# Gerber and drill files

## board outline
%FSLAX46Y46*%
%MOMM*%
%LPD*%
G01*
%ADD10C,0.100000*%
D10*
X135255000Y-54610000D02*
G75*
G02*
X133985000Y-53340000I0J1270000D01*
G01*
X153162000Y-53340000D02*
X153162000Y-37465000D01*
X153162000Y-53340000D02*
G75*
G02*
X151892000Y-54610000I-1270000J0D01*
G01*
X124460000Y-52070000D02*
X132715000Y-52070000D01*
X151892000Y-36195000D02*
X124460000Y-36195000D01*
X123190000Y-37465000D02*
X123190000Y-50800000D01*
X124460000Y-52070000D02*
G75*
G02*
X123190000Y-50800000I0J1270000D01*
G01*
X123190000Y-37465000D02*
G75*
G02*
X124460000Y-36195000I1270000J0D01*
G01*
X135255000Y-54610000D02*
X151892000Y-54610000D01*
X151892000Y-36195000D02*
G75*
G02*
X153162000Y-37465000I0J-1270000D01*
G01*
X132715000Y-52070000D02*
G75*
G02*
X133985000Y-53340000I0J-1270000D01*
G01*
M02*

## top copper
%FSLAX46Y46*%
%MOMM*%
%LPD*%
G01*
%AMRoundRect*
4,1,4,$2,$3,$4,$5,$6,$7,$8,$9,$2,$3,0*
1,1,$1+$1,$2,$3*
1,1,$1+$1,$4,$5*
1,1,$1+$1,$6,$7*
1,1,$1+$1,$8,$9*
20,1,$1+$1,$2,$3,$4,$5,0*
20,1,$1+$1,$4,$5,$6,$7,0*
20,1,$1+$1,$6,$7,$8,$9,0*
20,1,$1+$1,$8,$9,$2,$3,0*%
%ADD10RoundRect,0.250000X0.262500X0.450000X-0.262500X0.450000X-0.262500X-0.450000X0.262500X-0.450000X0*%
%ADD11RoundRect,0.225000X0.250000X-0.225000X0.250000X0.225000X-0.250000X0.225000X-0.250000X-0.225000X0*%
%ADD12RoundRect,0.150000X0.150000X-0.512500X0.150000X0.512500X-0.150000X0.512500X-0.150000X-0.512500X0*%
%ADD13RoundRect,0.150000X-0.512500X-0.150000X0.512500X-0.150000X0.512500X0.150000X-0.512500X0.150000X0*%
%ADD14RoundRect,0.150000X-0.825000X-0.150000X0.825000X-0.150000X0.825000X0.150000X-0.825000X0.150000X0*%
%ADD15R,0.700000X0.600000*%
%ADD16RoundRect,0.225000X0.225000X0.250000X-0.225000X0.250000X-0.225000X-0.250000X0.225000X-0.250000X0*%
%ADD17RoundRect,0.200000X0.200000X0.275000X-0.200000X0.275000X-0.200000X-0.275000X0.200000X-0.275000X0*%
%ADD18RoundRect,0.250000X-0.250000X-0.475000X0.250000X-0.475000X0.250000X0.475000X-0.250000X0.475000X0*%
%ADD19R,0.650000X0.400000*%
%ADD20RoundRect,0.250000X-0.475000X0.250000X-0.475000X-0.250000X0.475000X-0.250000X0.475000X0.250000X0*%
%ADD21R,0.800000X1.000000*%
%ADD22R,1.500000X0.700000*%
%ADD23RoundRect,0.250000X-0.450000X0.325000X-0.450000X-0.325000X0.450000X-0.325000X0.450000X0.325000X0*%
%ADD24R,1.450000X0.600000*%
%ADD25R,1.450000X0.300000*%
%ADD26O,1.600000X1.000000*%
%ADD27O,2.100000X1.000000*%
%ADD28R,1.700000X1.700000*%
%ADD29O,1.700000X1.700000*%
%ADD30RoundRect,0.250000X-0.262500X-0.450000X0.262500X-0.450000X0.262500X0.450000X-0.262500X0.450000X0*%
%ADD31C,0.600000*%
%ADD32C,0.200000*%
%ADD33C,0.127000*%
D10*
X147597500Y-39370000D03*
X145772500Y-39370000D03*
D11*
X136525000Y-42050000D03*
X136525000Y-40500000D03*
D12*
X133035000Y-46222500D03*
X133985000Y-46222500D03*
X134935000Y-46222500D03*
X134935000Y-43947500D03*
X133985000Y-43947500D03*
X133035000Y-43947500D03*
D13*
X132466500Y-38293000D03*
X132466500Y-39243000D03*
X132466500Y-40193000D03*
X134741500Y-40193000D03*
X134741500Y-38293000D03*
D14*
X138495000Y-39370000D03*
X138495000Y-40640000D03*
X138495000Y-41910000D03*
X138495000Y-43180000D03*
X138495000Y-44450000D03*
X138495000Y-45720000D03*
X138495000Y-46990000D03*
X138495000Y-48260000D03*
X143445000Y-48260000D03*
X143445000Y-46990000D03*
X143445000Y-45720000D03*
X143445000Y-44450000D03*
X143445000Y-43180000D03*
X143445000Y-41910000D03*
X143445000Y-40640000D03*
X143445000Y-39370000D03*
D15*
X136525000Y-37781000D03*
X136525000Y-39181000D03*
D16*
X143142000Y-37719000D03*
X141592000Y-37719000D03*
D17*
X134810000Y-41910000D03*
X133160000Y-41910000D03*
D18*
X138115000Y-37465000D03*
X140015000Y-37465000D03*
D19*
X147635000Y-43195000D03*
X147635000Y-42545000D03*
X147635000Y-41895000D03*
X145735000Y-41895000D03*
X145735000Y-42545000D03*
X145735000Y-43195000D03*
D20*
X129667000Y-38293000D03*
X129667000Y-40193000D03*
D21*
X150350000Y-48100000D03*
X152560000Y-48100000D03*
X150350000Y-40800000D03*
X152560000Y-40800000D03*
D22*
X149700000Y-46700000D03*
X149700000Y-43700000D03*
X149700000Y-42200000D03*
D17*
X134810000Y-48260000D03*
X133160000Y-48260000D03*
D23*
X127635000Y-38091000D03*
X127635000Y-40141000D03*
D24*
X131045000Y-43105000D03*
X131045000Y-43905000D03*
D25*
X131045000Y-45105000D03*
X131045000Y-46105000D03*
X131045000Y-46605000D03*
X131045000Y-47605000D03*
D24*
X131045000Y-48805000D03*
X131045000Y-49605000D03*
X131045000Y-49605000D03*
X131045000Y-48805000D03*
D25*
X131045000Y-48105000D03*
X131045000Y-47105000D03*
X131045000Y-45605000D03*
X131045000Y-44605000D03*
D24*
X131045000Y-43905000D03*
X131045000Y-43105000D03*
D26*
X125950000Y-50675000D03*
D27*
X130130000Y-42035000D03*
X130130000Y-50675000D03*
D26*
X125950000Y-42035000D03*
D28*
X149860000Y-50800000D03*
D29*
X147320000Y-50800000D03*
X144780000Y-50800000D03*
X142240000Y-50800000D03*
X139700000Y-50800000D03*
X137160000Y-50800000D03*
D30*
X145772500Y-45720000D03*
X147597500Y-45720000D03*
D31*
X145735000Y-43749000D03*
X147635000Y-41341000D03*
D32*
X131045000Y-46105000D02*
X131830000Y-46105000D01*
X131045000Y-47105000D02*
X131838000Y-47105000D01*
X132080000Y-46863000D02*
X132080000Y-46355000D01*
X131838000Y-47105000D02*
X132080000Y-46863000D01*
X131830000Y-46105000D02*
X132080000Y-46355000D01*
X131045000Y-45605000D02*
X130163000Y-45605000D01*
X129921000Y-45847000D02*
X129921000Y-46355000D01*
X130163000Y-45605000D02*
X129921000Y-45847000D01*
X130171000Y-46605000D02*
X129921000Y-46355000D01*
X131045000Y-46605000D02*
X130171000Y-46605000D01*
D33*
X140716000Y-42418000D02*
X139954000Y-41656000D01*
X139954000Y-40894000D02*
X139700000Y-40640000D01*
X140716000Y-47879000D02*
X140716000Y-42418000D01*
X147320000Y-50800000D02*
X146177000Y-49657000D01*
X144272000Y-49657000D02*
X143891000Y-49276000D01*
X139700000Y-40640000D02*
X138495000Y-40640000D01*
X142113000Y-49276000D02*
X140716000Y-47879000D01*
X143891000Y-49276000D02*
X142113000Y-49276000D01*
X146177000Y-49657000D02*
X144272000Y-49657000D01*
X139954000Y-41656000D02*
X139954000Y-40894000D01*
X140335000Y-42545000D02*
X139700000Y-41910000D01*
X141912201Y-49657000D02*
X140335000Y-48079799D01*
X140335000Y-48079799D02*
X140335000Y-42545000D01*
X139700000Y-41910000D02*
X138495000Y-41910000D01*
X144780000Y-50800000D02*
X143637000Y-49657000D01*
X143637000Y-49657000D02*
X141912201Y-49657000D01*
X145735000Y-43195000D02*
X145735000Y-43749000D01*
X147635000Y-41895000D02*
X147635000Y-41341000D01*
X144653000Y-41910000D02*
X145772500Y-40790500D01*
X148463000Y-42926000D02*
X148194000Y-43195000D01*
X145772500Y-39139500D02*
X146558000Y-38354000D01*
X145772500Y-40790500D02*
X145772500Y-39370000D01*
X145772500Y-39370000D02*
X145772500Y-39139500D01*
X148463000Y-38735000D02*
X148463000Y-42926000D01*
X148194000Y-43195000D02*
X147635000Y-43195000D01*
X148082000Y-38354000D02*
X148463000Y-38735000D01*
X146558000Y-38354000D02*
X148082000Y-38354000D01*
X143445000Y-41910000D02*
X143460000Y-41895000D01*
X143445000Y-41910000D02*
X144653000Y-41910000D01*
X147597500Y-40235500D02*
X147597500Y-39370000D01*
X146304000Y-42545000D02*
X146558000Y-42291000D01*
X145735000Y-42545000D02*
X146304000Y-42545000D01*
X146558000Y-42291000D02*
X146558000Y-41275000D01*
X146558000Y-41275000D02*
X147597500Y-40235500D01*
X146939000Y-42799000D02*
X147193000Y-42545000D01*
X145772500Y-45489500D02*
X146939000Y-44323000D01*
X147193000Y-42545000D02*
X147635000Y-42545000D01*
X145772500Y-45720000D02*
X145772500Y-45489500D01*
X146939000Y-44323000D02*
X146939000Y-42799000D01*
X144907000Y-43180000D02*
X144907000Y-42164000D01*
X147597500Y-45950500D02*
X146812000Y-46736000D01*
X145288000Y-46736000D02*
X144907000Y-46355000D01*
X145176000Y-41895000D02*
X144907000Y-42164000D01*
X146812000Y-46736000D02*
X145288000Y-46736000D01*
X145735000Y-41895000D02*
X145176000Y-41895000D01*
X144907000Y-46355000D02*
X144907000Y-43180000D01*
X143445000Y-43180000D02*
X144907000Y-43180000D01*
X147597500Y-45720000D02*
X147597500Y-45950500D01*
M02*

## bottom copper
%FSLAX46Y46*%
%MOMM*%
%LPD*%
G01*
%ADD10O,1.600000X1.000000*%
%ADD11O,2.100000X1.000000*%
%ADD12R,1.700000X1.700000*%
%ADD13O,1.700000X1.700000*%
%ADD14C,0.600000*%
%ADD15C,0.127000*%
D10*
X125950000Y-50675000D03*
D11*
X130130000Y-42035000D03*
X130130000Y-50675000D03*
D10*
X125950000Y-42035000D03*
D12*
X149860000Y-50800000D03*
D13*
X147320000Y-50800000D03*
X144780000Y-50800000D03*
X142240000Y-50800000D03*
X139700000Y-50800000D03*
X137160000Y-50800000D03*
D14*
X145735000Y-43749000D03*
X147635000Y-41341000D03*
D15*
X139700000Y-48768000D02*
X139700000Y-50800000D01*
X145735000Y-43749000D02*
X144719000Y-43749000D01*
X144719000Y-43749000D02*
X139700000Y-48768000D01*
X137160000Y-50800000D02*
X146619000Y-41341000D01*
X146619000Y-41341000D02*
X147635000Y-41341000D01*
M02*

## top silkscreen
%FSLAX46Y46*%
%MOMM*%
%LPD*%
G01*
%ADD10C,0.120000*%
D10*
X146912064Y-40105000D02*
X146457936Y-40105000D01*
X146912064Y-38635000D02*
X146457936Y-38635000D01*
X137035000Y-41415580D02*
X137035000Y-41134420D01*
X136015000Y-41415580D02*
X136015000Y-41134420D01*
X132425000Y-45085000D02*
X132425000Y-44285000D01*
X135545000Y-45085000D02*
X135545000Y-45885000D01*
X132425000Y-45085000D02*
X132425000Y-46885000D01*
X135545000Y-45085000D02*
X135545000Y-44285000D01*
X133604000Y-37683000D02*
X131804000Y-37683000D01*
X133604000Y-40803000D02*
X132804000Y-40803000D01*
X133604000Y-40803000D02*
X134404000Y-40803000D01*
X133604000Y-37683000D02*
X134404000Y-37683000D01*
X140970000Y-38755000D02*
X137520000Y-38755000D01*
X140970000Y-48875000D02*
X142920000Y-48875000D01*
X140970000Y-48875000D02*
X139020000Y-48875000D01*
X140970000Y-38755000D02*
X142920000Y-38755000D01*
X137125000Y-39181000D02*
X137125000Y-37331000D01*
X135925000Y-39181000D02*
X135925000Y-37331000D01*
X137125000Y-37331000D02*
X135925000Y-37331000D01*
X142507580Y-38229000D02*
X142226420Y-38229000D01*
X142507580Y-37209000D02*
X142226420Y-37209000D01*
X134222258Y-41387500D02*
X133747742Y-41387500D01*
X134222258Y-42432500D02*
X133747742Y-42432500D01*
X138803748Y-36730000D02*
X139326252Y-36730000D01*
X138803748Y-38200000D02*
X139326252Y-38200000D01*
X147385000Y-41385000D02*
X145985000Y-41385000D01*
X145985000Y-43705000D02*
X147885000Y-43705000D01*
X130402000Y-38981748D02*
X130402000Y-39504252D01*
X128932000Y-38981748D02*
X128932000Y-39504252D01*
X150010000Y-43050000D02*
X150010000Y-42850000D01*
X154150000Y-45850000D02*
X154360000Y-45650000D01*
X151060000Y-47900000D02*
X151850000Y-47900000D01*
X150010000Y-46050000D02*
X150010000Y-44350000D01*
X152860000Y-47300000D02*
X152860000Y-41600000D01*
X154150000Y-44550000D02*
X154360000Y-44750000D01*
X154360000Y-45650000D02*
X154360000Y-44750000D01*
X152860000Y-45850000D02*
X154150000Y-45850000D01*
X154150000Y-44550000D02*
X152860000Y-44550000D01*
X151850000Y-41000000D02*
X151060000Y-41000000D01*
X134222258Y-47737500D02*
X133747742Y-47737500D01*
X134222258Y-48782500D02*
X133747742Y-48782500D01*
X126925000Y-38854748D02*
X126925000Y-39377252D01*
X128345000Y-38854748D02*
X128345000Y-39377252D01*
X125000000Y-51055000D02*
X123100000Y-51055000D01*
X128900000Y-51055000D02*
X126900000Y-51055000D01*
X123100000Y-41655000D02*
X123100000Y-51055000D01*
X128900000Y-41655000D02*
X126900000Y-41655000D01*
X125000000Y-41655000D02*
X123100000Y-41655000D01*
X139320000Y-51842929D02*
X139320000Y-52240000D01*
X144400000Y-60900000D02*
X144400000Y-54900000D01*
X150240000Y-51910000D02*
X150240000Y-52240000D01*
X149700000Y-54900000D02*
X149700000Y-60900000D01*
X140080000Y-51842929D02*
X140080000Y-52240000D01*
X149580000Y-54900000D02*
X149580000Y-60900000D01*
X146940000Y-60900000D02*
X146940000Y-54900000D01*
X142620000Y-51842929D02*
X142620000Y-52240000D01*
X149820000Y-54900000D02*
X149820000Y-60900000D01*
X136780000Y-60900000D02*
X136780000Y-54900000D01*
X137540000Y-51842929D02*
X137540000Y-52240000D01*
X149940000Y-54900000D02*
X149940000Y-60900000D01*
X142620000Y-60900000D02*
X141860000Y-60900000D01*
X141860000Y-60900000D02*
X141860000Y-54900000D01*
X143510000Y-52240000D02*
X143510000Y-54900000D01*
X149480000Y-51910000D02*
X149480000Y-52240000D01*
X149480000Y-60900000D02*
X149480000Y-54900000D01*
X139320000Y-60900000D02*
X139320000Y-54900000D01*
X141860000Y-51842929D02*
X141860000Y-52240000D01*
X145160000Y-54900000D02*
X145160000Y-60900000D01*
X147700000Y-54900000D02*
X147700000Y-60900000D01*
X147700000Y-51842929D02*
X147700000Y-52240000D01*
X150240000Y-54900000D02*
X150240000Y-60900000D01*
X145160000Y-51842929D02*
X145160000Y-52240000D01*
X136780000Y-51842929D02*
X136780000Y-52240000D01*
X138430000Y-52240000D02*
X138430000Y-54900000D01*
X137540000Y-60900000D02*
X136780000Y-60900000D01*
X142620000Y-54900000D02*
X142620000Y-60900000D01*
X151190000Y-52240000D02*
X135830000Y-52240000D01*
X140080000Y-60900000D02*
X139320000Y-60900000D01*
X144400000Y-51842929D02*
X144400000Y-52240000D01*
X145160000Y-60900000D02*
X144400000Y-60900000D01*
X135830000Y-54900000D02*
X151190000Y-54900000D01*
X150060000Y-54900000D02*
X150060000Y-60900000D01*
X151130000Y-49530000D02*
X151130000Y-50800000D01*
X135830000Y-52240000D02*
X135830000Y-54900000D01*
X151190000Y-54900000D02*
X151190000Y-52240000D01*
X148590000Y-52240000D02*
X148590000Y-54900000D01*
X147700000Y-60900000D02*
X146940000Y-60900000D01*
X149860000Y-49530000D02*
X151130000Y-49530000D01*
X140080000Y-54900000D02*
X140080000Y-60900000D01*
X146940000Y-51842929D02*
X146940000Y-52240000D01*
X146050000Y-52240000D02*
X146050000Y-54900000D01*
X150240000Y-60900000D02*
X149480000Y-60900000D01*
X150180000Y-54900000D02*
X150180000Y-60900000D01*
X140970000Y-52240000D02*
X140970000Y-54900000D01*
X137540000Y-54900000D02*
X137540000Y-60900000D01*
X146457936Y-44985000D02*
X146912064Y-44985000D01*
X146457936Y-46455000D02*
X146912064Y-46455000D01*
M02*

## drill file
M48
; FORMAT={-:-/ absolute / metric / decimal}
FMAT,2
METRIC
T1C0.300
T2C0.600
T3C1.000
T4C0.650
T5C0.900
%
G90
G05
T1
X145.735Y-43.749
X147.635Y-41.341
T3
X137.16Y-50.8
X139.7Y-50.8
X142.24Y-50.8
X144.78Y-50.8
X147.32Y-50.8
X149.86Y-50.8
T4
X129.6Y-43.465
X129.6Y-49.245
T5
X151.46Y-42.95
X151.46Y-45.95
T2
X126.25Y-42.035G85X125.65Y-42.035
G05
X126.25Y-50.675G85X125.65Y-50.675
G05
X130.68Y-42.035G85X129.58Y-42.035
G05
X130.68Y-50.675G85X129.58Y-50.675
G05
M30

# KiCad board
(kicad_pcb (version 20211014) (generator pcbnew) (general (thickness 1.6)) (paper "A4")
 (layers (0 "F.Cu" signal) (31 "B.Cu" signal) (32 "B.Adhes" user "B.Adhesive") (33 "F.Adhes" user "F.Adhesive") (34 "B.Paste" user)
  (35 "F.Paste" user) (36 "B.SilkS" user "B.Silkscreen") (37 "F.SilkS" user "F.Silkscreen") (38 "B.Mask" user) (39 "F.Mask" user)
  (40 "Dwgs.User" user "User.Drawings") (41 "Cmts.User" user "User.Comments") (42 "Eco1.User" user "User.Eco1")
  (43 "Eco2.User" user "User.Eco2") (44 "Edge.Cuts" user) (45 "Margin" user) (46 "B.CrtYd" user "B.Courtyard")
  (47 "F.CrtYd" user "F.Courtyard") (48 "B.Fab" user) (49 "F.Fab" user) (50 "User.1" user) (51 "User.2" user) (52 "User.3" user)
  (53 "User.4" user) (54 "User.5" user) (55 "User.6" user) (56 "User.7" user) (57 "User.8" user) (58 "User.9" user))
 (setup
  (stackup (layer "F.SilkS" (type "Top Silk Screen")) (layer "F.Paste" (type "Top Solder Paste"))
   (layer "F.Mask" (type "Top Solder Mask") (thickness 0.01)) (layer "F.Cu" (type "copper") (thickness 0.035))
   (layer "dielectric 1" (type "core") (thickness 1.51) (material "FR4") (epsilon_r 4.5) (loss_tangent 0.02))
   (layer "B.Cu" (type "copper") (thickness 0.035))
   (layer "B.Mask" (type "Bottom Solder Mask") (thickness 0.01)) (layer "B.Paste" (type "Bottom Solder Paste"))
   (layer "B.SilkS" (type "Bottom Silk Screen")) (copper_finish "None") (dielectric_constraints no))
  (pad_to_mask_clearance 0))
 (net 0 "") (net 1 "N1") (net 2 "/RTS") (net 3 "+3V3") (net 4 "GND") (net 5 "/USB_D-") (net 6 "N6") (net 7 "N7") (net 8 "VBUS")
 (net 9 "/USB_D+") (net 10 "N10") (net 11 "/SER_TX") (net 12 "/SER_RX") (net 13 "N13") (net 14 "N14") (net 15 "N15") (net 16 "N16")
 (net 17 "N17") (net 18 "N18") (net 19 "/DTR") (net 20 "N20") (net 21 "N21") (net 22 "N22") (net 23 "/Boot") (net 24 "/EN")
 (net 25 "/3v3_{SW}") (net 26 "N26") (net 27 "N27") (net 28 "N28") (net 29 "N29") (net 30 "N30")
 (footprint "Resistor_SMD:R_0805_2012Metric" (layer "F.Cu") (at 146.685 39.37 180)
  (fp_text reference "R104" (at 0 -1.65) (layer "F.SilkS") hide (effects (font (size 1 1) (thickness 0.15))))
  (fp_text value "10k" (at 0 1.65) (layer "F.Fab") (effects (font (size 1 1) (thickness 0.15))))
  (fp_line (start -0.227064 -0.735) (end 0.227064 -0.735) (layer "F.SilkS") (width 0.12))
  (fp_line (start -0.227064 0.735) (end 0.227064 0.735) (layer "F.SilkS") (width 0.12))
  (pad "1" smd roundrect locked (at -0.9125 0 180) (size 1.025 1.4) (layers "F.Cu" "F.Paste" "F.Mask") (roundrect_rratio 0.243902)
   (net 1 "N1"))
  (pad "2" smd roundrect locked (at 0.9125 0 180) (size 1.025 1.4) (layers "F.Cu" "F.Paste" "F.Mask") (roundrect_rratio 0.243902)
   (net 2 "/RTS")))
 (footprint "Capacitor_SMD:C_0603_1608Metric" (layer "F.Cu") (at 136.525 41.275 90) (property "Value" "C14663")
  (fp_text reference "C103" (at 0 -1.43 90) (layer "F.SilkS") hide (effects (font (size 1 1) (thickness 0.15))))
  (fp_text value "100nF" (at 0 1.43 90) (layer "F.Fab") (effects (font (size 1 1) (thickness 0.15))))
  (fp_line (start -0.14058 0.51) (end 0.14058 0.51) (layer "F.SilkS") (width 0.12))
  (fp_line (start -0.14058 -0.51) (end 0.14058 -0.51) (layer "F.SilkS") (width 0.12))
  (pad "1" smd roundrect locked (at -0.775 0 90) (size 0.9 0.95) (layers "F.Cu" "F.Paste" "F.Mask") (roundrect_rratio 0.25) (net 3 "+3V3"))
  (pad "2" smd roundrect locked (at 0.775 0 90) (size 0.9 0.95) (layers "F.Cu" "F.Paste" "F.Mask") (roundrect_rratio 0.25) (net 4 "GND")))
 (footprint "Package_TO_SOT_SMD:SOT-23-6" (layer "F.Cu") (at 133.985 45.085 90)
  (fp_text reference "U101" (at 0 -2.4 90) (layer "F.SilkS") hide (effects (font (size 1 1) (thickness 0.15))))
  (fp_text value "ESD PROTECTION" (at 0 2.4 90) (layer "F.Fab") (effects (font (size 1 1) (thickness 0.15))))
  (fp_line (start 0 -1.56) (end 0.8 -1.56) (layer "F.SilkS") (width 0.12))
  (fp_line (start 0 1.56) (end -0.8 1.56) (layer "F.SilkS") (width 0.12))
  (fp_line (start 0 -1.56) (end -1.8 -1.56) (layer "F.SilkS") (width 0.12))
  (fp_line (start 0 1.56) (end 0.8 1.56) (layer "F.SilkS") (width 0.12))
  (pad "1" smd roundrect locked (at -1.1375 -0.95 90) (size 1.325 0.6) (layers "F.Cu" "F.Paste" "F.Mask") (roundrect_rratio 0.25)
   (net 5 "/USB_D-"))
  (pad "2" smd roundrect locked (at -1.1375 0 90) (size 1.325 0.6) (layers "F.Cu" "F.Paste" "F.Mask") (roundrect_rratio 0.25) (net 4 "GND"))
  (pad "3" smd roundrect locked (at -1.1375 0.95 90) (size 1.325 0.6) (layers "F.Cu" "F.Paste" "F.Mask") (roundrect_rratio 0.25)
   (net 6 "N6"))
  (pad "4" smd roundrect locked (at 1.1375 0.95 90) (size 1.325 0.6) (layers "F.Cu" "F.Paste" "F.Mask") (roundrect_rratio 0.25) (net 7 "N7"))
  (pad "5" smd roundrect locked (at 1.1375 0 90) (size 1.325 0.6) (layers "F.Cu" "F.Paste" "F.Mask") (roundrect_rratio 0.25) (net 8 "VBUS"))
  (pad "6" smd roundrect locked (at 1.1375 -0.95 90) (size 1.325 0.6) (layers "F.Cu" "F.Paste" "F.Mask") (roundrect_rratio 0.25)
   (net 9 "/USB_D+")))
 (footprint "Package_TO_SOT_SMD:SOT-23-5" (layer "F.Cu") (at 133.604 39.243)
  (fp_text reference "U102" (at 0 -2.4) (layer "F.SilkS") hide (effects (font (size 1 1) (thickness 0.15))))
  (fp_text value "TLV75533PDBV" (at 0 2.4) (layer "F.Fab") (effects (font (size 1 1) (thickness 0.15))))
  (fp_line (start 0 -1.56) (end -1.8 -1.56) (layer "F.SilkS") (width 0.12))
  (fp_line (start 0 1.56) (end -0.8 1.56) (layer "F.SilkS") (width 0.12))
  (fp_line (start 0 1.56) (end 0.8 1.56) (layer "F.SilkS") (width 0.12))
  (fp_line (start 0 -1.56) (end 0.8 -1.56) (layer "F.SilkS") (width 0.12))
  (pad "1" smd roundrect locked (at -1.1375 -0.95) (size 1.325 0.6) (layers "F.Cu" "F.Paste" "F.Mask") (roundrect_rratio 0.25)
   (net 8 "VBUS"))
  (pad "2" smd roundrect locked (at -1.1375 0) (size 1.325 0.6) (layers "F.Cu" "F.Paste" "F.Mask") (roundrect_rratio 0.25) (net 4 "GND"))
  (pad "3" smd roundrect locked (at -1.1375 0.95) (size 1.325 0.6) (layers "F.Cu" "F.Paste" "F.Mask") (roundrect_rratio 0.25) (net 8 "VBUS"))
  (pad "4" smd roundrect locked (at 1.1375 0.95) (size 1.325 0.6) (layers "F.Cu" "F.Paste" "F.Mask") (roundrect_rratio 0.25) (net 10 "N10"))
  (pad "5" smd roundrect locked (at 1.1375 -0.95) (size 1.325 0.6) (layers "F.Cu" "F.Paste" "F.Mask") (roundrect_rratio 0.25) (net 3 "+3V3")))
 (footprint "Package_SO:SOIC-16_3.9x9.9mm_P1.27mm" (layer "F.Cu") (at 140.97 43.815)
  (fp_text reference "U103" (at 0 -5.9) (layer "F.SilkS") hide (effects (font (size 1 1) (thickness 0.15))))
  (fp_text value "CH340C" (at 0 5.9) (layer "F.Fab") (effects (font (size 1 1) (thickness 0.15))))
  (fp_line (start 0 -5.06) (end -3.45 -5.06) (layer "F.SilkS") (width 0.12))
  (fp_line (start 0 5.06) (end 1.95 5.06) (layer "F.SilkS") (width 0.12))
  (fp_line (start 0 5.06) (end -1.95 5.06) (layer "F.SilkS") (width 0.12))
  (fp_line (start 0 -5.06) (end 1.95 -5.06) (layer "F.SilkS") (width 0.12))
  (pad "1" smd roundrect locked (at -2.475 -4.445) (size 1.95 0.6) (layers "F.Cu" "F.Paste" "F.Mask") (roundrect_rratio 0.25) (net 4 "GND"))
  (pad "2" smd roundrect locked (at -2.475 -3.175) (size 1.95 0.6) (layers "F.Cu" "F.Paste" "F.Mask") (roundrect_rratio 0.25)
   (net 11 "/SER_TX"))
  (pad "3" smd roundrect locked (at -2.475 -1.905) (size 1.95 0.6) (layers "F.Cu" "F.Paste" "F.Mask") (roundrect_rratio 0.25)
   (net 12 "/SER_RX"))
  (pad "4" smd roundrect locked (at -2.475 -0.635) (size 1.95 0.6) (layers "F.Cu" "F.Paste" "F.Mask") (roundrect_rratio 0.25) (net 3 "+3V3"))
  (pad "5" smd roundrect locked (at -2.475 0.635) (size 1.95 0.6) (layers "F.Cu" "F.Paste" "F.Mask") (roundrect_rratio 0.25)
   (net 9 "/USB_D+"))
  (pad "6" smd roundrect locked (at -2.475 1.905) (size 1.95 0.6) (layers "F.Cu" "F.Paste" "F.Mask") (roundrect_rratio 0.25)
   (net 5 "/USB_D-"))
  (pad "7" smd roundrect locked (at -2.475 3.175) (size 1.95 0.6) (layers "F.Cu" "F.Paste" "F.Mask") (roundrect_rratio 0.25) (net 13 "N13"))
  (pad "8" smd roundrect locked (at -2.475 4.445) (size 1.95 0.6) (layers "F.Cu" "F.Paste" "F.Mask") (roundrect_rratio 0.25) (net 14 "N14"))
  (pad "9" smd roundrect locked (at 2.475 4.445) (size 1.95 0.6) (layers "F.Cu" "F.Paste" "F.Mask") (roundrect_rratio 0.25) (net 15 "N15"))
  (pad "10" smd roundrect locked (at 2.475 3.175) (size 1.95 0.6) (layers "F.Cu" "F.Paste" "F.Mask") (roundrect_rratio 0.25) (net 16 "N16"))
  (pad "11" smd roundrect locked (at 2.475 1.905) (size 1.95 0.6) (layers "F.Cu" "F.Paste" "F.Mask") (roundrect_rratio 0.25) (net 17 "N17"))
  (pad "12" smd roundrect locked (at 2.475 0.635) (size 1.95 0.6) (layers "F.Cu" "F.Paste" "F.Mask") (roundrect_rratio 0.25) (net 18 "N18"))
  (pad "13" smd roundrect locked (at 2.475 -0.635) (size 1.95 0.6) (layers "F.Cu" "F.Paste" "F.Mask") (roundrect_rratio 0.25)
   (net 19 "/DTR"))
  (pad "14" smd roundrect locked (at 2.475 -1.905) (size 1.95 0.6) (layers "F.Cu" "F.Paste" "F.Mask") (roundrect_rratio 0.25) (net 2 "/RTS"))
  (pad "15" smd roundrect locked (at 2.475 -3.175) (size 1.95 0.6) (layers "F.Cu" "F.Paste" "F.Mask") (roundrect_rratio 0.25) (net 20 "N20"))
  (pad "16" smd roundrect locked (at 2.475 -4.445) (size 1.95 0.6) (layers "F.Cu" "F.Paste" "F.Mask") (roundrect_rratio 0.25) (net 3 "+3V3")))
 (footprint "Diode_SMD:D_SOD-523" (layer "F.Cu") (at 136.525 38.481 -90)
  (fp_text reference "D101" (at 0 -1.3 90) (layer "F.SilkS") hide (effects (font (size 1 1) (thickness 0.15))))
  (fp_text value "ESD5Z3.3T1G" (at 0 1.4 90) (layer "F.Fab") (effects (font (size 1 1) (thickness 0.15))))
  (fp_line (start 0.7 -0.6) (end -1.15 -0.6) (layer "F.SilkS") (width 0.12))
  (fp_line (start 0.7 0.6) (end -1.15 0.6) (layer "F.SilkS") (width 0.12))
  (fp_line (start -1.15 -0.6) (end -1.15 0.6) (layer "F.SilkS") (width 0.12))
  (pad "1" smd rect locked (at -0.7 0 90) (size 0.6 0.7) (layers "F.Cu" "F.Paste" "F.Mask") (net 3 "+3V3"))
  (pad "2" smd rect locked (at 0.7 0 90) (size 0.6 0.7) (layers "F.Cu" "F.Paste" "F.Mask") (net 4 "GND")))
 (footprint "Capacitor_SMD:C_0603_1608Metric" (layer "F.Cu") (at 142.367 37.719 180) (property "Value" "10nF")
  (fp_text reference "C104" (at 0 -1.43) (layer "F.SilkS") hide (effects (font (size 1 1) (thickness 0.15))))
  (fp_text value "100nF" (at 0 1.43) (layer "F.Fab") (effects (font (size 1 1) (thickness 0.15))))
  (fp_line (start -0.14058 -0.51) (end 0.14058 -0.51) (layer "F.SilkS") (width 0.12))
  (fp_line (start -0.14058 0.51) (end 0.14058 0.51) (layer "F.SilkS") (width 0.12))
  (pad "1" smd roundrect locked (at -0.775 0 180) (size 0.9 0.95) (layers "F.Cu" "F.Paste" "F.Mask") (roundrect_rratio 0.25) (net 3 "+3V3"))
  (pad "2" smd roundrect locked (at 0.775 0 180) (size 0.9 0.95) (layers "F.Cu" "F.Paste" "F.Mask") (roundrect_rratio 0.25) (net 4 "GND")))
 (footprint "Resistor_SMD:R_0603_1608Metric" (layer "F.Cu") (at 133.985 41.91 180)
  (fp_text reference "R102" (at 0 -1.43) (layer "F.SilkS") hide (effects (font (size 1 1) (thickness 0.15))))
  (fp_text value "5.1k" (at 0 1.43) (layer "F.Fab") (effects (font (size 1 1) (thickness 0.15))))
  (fp_line (start -0.237258 0.5225) (end 0.237258 0.5225) (layer "F.SilkS") (width 0.12))
  (fp_line (start -0.237258 -0.5225) (end 0.237258 -0.5225) (layer "F.SilkS") (width 0.12))
  (pad "1" smd roundrect locked (at -0.825 0 180) (size 0.8 0.95) (layers "F.Cu" "F.Paste" "F.Mask") (roundrect_rratio 0.25) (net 4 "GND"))
  (pad "2" smd roundrect locked (at 0.825 0 180) (size 0.8 0.95) (layers "F.Cu" "F.Paste" "F.Mask") (roundrect_rratio 0.25) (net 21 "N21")))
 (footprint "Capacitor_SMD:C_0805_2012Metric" (layer "F.Cu") (at 139.065 37.465)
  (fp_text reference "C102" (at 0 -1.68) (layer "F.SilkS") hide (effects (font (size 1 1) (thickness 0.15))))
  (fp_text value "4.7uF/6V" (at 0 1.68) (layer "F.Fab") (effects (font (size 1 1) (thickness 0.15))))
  (fp_line (start -0.261252 -0.735) (end 0.261252 -0.735) (layer "F.SilkS") (width 0.12))
  (fp_line (start -0.261252 0.735) (end 0.261252 0.735) (layer "F.SilkS") (width 0.12))
  (pad "1" smd roundrect locked (at -0.95 0) (size 1 1.45) (layers "F.Cu" "F.Paste" "F.Mask") (roundrect_rratio 0.25) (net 3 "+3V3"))
  (pad "2" smd roundrect locked (at 0.95 0) (size 1 1.45) (layers "F.Cu" "F.Paste" "F.Mask") (roundrect_rratio 0.25) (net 4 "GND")))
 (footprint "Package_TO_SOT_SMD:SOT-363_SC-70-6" (layer "F.Cu") (at 146.685 42.545 180)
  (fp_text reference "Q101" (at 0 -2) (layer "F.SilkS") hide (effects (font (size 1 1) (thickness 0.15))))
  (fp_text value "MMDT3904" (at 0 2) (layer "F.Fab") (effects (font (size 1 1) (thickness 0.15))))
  (fp_line (start -0.7 1.16) (end 0.7 1.16) (layer "F.SilkS") (width 0.12))
  (fp_line (start 0.7 -1.16) (end -1.2 -1.16) (layer "F.SilkS") (width 0.12))
  (pad "1" smd rect locked (at -0.95 -0.65 180) (size 0.65 0.4) (layers "F.Cu" "F.Paste" "F.Mask") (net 2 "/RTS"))
  (pad "2" smd rect locked (at -0.95 0 180) (size 0.65 0.4) (layers "F.Cu" "F.Paste" "F.Mask") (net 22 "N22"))
  (pad "3" smd rect locked (at -0.95 0.65 180) (size 0.65 0.4) (layers "F.Cu" "F.Paste" "F.Mask") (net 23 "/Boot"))
  (pad "4" smd rect locked (at 0.95 0.65 180) (size 0.65 0.4) (layers "F.Cu" "F.Paste" "F.Mask") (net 19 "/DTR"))
  (pad "5" smd rect locked (at 0.95 0 180) (size 0.65 0.4) (layers "F.Cu" "F.Paste" "F.Mask") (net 1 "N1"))
  (pad "6" smd rect locked (at 0.95 -0.65 180) (size 0.65 0.4) (layers "F.Cu" "F.Paste" "F.Mask") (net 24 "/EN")))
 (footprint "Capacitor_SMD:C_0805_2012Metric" (layer "F.Cu") (at 129.667 39.243 -90)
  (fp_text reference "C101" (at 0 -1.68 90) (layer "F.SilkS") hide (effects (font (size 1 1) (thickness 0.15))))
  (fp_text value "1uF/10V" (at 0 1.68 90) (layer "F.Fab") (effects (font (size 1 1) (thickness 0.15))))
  (fp_line (start -0.261252 -0.735) (end 0.261252 -0.735) (layer "F.SilkS") (width 0.12))
  (fp_line (start -0.261252 0.735) (end 0.261252 0.735) (layer "F.SilkS") (width 0.12))
  (pad "1" smd roundrect locked (at -0.95 0 270) (size 1 1.45) (layers "F.Cu" "F.Paste" "F.Mask") (roundrect_rratio 0.25) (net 8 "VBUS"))
  (pad "2" smd roundrect locked (at 0.95 0 270) (size 1 1.45) (layers "F.Cu" "F.Paste" "F.Mask") (roundrect_rratio 0.25) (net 4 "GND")))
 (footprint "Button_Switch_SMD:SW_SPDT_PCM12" (layer "F.Cu") (at 151.13 44.45 90)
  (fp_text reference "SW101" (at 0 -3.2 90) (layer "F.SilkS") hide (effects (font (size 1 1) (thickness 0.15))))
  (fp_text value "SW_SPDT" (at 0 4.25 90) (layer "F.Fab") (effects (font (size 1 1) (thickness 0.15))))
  (fp_line (start 1.4 -1.12) (end 1.6 -1.12) (layer "F.SilkS") (width 0.12))
  (fp_line (start -1.4 3.02) (end -1.2 3.23) (layer "F.SilkS") (width 0.12))
  (fp_line (start -3.45 -0.07) (end -3.45 0.72) (layer "F.SilkS") (width 0.12))
  (fp_line (start -1.6 -1.12) (end 0.1 -1.12) (layer "F.SilkS") (width 0.12))
  (fp_line (start -2.85 1.73) (end 2.85 1.73) (layer "F.SilkS") (width 0.12))
  (fp_line (start -0.1 3.02) (end -0.3 3.23) (layer "F.SilkS") (width 0.12))
  (fp_line (start -1.2 3.23) (end -0.3 3.23) (layer "F.SilkS") (width 0.12))
  (fp_line (start -1.4 1.73) (end -1.4 3.02) (layer "F.SilkS") (width 0.12))
  (fp_line (start -0.1 3.02) (end -0.1 1.73) (layer "F.SilkS") (width 0.12))
  (fp_line (start 3.45 0.72) (end 3.45 -0.07) (layer "F.SilkS") (width 0.12))
  (pad "" smd rect locked (at -3.65 -0.78 90) (size 1 0.8) (layers "F.Cu" "F.Paste" "F.Mask"))
  (pad "" np_thru_hole circle locked (at -1.5 0.33 90) (size 0.9 0.9) (drill 0.9) (layers *.Cu *.Mask))
  (pad "" smd rect locked (at -3.65 1.43 90) (size 1 0.8) (layers "F.Cu" "F.Paste" "F.Mask"))
  (pad "" smd rect locked (at 3.65 -0.78 90) (size 1 0.8) (layers "F.Cu" "F.Paste" "F.Mask"))
  (pad "" smd rect locked (at 3.65 1.43 90) (size 1 0.8) (layers "F.Cu" "F.Paste" "F.Mask"))
  (pad "" np_thru_hole circle locked (at 1.5 0.33 90) (size 0.9 0.9) (drill 0.9) (layers *.Cu *.Mask))
  (pad "1" smd rect locked (at -2.25 -1.43 90) (size 0.7 1.5) (layers "F.Cu" "F.Paste" "F.Mask") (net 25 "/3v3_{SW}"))
  (pad "2" smd rect locked (at 0.75 -1.43 90) (size 0.7 1.5) (layers "F.Cu" "F.Paste" "F.Mask") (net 3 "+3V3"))
  (pad "3" smd rect locked (at 2.25 -1.43 90) (size 0.7 1.5) (layers "F.Cu" "F.Paste" "F.Mask") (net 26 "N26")))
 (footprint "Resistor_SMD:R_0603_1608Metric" (layer "F.Cu") (at 133.985 48.26 180)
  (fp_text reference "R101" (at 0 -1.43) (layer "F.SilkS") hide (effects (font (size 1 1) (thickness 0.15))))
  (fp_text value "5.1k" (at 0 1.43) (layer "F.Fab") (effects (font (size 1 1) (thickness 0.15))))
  (fp_line (start -0.237258 0.5225) (end 0.237258 0.5225) (layer "F.SilkS") (width 0.12))
  (fp_line (start -0.237258 -0.5225) (end 0.237258 -0.5225) (layer "F.SilkS") (width 0.12))
  (pad "1" smd roundrect locked (at -0.825 0 180) (size 0.8 0.95) (layers "F.Cu" "F.Paste" "F.Mask") (roundrect_rratio 0.25) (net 4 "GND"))
  (pad "2" smd roundrect locked (at 0.825 0 180) (size 0.8 0.95) (layers "F.Cu" "F.Paste" "F.Mask") (roundrect_rratio 0.25) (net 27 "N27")))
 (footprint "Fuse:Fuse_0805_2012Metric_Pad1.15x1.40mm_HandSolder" (layer "F.Cu") (at 127.635 39.116 -90)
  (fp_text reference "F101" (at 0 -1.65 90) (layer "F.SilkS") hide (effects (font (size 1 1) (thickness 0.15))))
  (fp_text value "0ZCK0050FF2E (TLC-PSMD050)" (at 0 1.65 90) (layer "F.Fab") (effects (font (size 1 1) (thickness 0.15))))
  (fp_line (start -0.261252 0.71) (end 0.261252 0.71) (layer "F.SilkS") (width 0.12))
  (fp_line (start -0.261252 -0.71) (end 0.261252 -0.71) (layer "F.SilkS") (width 0.12))
  (pad "1" smd roundrect locked (at -1.025 0 270) (size 1.15 1.4) (layers "F.Cu" "F.Paste" "F.Mask") (roundrect_rratio 0.217391)
   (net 8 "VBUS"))
  (pad "2" smd roundrect locked (at 1.025 0 270) (size 1.15 1.4) (layers "F.Cu" "F.Paste" "F.Mask") (roundrect_rratio 0.217391)
   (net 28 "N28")))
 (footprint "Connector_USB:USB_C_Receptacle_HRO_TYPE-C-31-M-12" (layer "F.Cu") (at 127 46.355 -90)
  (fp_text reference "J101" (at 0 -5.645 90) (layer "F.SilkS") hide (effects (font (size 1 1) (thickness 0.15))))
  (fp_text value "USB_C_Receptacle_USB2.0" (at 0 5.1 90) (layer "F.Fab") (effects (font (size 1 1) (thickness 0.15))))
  (fp_line (start 4.7 2) (end 4.7 3.9) (layer "F.SilkS") (width 0.12))
  (fp_line (start 4.7 -1.9) (end 4.7 0.1) (layer "F.SilkS") (width 0.12))
  (fp_line (start -4.7 3.9) (end 4.7 3.9) (layer "F.SilkS") (width 0.12))
  (fp_line (start -4.7 -1.9) (end -4.7 0.1) (layer "F.SilkS") (width 0.12))
  (fp_line (start -4.7 2) (end -4.7 3.9) (layer "F.SilkS") (width 0.12))
  (pad "" np_thru_hole circle locked (at 2.89 -2.6 270) (size 0.65 0.65) (drill 0.65) (layers *.Cu *.Mask))
  (pad "" np_thru_hole circle locked (at -2.89 -2.6 270) (size 0.65 0.65) (drill 0.65) (layers *.Cu *.Mask))
  (pad "A1" smd rect locked (at -3.25 -4.045 270) (size 0.6 1.45) (layers "F.Cu" "F.Paste" "F.Mask") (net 4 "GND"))
  (pad "A4" smd rect locked (at -2.45 -4.045 270) (size 0.6 1.45) (layers "F.Cu" "F.Paste" "F.Mask") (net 28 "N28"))
  (pad "A5" smd rect locked (at -1.25 -4.045 270) (size 0.3 1.45) (layers "F.Cu" "F.Paste" "F.Mask") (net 21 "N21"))
  (pad "A6" smd rect locked (at -0.25 -4.045 270) (size 0.3 1.45) (layers "F.Cu" "F.Paste" "F.Mask") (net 9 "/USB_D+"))
  (pad "A7" smd rect locked (at 0.25 -4.045 270) (size 0.3 1.45) (layers "F.Cu" "F.Paste" "F.Mask") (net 5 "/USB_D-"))
  (pad "A8" smd rect locked (at 1.25 -4.045 270) (size 0.3 1.45) (layers "F.Cu" "F.Paste" "F.Mask") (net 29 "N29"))
  (pad "A9" smd rect locked (at 2.45 -4.045 270) (size 0.6 1.45) (layers "F.Cu" "F.Paste" "F.Mask") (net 28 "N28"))
  (pad "A12" smd rect locked (at 3.25 -4.045 270) (size 0.6 1.45) (layers "F.Cu" "F.Paste" "F.Mask") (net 4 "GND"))
  (pad "B1" smd rect locked (at 3.25 -4.045 270) (size 0.6 1.45) (layers "F.Cu" "F.Paste" "F.Mask") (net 4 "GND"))
  (pad "B4" smd rect locked (at 2.45 -4.045 270) (size 0.6 1.45) (layers "F.Cu" "F.Paste" "F.Mask") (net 28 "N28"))
  (pad "B5" smd rect locked (at 1.75 -4.045 270) (size 0.3 1.45) (layers "F.Cu" "F.Paste" "F.Mask") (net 27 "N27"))
  (pad "B6" smd rect locked (at 0.75 -4.045 270) (size 0.3 1.45) (layers "F.Cu" "F.Paste" "F.Mask") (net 9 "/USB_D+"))
  (pad "B7" smd rect locked (at -0.75 -4.045 270) (size 0.3 1.45) (layers "F.Cu" "F.Paste" "F.Mask") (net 5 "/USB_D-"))
  (pad "B8" smd rect locked (at -1.75 -4.045 270) (size 0.3 1.45) (layers "F.Cu" "F.Paste" "F.Mask") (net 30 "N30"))
  (pad "B9" smd rect locked (at -2.45 -4.045 270) (size 0.6 1.45) (layers "F.Cu" "F.Paste" "F.Mask") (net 28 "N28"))
  (pad "B12" smd rect locked (at -3.25 -4.045 270) (size 0.6 1.45) (layers "F.Cu" "F.Paste" "F.Mask") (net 4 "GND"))
  (pad "S1" thru_hole oval locked (at 4.32 1.05 270) (size 1 1.6) (drill oval 0.6 1.2) (layers *.Cu *.Mask) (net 4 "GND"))
  (pad "S1" thru_hole oval locked (at -4.32 -3.13 270) (size 1 2.1) (drill oval 0.6 1.7) (layers *.Cu *.Mask) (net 4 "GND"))
  (pad "S1" thru_hole oval locked (at 4.32 -3.13 270) (size 1 2.1) (drill oval 0.6 1.7) (layers *.Cu *.Mask) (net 4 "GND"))
  (pad "S1" thru_hole oval locked (at -4.32 1.05 270) (size 1 1.6) (drill oval 0.6 1.2) (layers *.Cu *.Mask) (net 4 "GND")))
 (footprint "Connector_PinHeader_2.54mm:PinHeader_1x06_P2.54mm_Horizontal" (layer "F.Cu") (at 149.86 50.8 -90)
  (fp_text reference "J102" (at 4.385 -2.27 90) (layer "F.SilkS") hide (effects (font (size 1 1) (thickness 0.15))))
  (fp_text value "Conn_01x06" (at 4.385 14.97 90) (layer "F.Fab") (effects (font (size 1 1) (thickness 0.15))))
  (fp_line (start 1.042929 10.54) (end 1.44 10.54) (layer "F.SilkS") (width 0.12))
  (fp_line (start 10.1 5.46) (end 4.1 5.46) (layer "F.SilkS") (width 0.12))
  (fp_line (start 1.11 -0.38) (end 1.44 -0.38) (layer "F.SilkS") (width 0.12))
  (fp_line (start 4.1 0.16) (end 10.1 0.16) (layer "F.SilkS") (width 0.12))
  (fp_line (start 1.042929 9.78) (end 1.44 9.78) (layer "F.SilkS") (width 0.12))
  (fp_line (start 4.1 0.28) (end 10.1 0.28) (layer "F.SilkS") (width 0.12))
  (fp_line (start 10.1 2.92) (end 4.1 2.92) (layer "F.SilkS") (width 0.12))
  (fp_line (start 1.042929 7.24) (end 1.44 7.24) (layer "F.SilkS") (width 0.12))
  (fp_line (start 4.1 0.04) (end 10.1 0.04) (layer "F.SilkS") (width 0.12))
  (fp_line (start 10.1 13.08) (end 4.1 13.08) (layer "F.SilkS") (width 0.12))
  (fp_line (start 1.042929 12.32) (end 1.44 12.32) (layer "F.SilkS") (width 0.12))
  (fp_line (start 4.1 -0.08) (end 10.1 -0.08) (layer "F.SilkS") (width 0.12))
  (fp_line (start 10.1 7.24) (end 10.1 8) (layer "F.SilkS") (width 0.12))
  (fp_line (start 10.1 8) (end 4.1 8) (layer "F.SilkS") (width 0.12))
  (fp_line (start 1.44 6.35) (end 4.1 6.35) (layer "F.SilkS") (width 0.12))
  (fp_line (start 1.11 0.38) (end 1.44 0.38) (layer "F.SilkS") (width 0.12))
  (fp_line (start 10.1 0.38) (end 4.1 0.38) (layer "F.SilkS") (width 0.12))
  (fp_line (start 10.1 10.54) (end 4.1 10.54) (layer "F.SilkS") (width 0.12))
  (fp_line (start 1.042929 8) (end 1.44 8) (layer "F.SilkS") (width 0.12))
  (fp_line (start 4.1 4.7) (end 10.1 4.7) (layer "F.SilkS") (width 0.12))
  (fp_line (start 4.1 2.16) (end 10.1 2.16) (layer "F.SilkS") (width 0.12))
  (fp_line (start 1.042929 2.16) (end 1.44 2.16) (layer "F.SilkS") (width 0.12))
  (fp_line (start 4.1 -0.38) (end 10.1 -0.38) (layer "F.SilkS") (width 0.12))
  (fp_line (start 1.042929 4.7) (end 1.44 4.7) (layer "F.SilkS") (width 0.12))
  (fp_line (start 1.042929 13.08) (end 1.44 13.08) (layer "F.SilkS") (width 0.12))
  (fp_line (start 1.44 11.43) (end 4.1 11.43) (layer "F.SilkS") (width 0.12))
  (fp_line (start 10.1 12.32) (end 10.1 13.08) (layer "F.SilkS") (width 0.12))
  (fp_line (start 4.1 7.24) (end 10.1 7.24) (layer "F.SilkS") (width 0.12))
  (fp_line (start 1.44 -1.33) (end 1.44 14.03) (layer "F.SilkS") (width 0.12))
  (fp_line (start 10.1 9.78) (end 10.1 10.54) (layer "F.SilkS") (width 0.12))
  (fp_line (start 1.042929 5.46) (end 1.44 5.46) (layer "F.SilkS") (width 0.12))
  (fp_line (start 10.1 4.7) (end 10.1 5.46) (layer "F.SilkS") (width 0.12))
  (fp_line (start 4.1 14.03) (end 4.1 -1.33) (layer "F.SilkS") (width 0.12))
  (fp_line (start 4.1 -0.2) (end 10.1 -0.2) (layer "F.SilkS") (width 0.12))
  (fp_line (start -1.27 -1.27) (end 0 -1.27) (layer "F.SilkS") (width 0.12))
  (fp_line (start 1.44 14.03) (end 4.1 14.03) (layer "F.SilkS") (width 0.12))
  (fp_line (start 4.1 -1.33) (end 1.44 -1.33) (layer "F.SilkS") (width 0.12))
  (fp_line (start 1.44 1.27) (end 4.1 1.27) (layer "F.SilkS") (width 0.12))
  (fp_line (start 10.1 2.16) (end 10.1 2.92) (layer "F.SilkS") (width 0.12))
  (fp_line (start -1.27 0) (end -1.27 -1.27) (layer "F.SilkS") (width 0.12))
  (fp_line (start 4.1 9.78) (end 10.1 9.78) (layer "F.SilkS") (width 0.12))
  (fp_line (start 1.042929 2.92) (end 1.44 2.92) (layer "F.SilkS") (width 0.12))
  (fp_line (start 1.44 3.81) (end 4.1 3.81) (layer "F.SilkS") (width 0.12))
  (fp_line (start 10.1 -0.38) (end 10.1 0.38) (layer "F.SilkS") (width 0.12))
  (fp_line (start 4.1 -0.32) (end 10.1 -0.32) (layer "F.SilkS") (width 0.12))
  (fp_line (start 1.44 8.89) (end 4.1 8.89) (layer "F.SilkS") (width 0.12))
  (fp_line (start 4.1 12.32) (end 10.1 12.32) (layer "F.SilkS") (width 0.12))
  (pad "1" thru_hole rect locked (at 0 0 270) (size 1.7 1.7) (drill 1) (layers *.Cu *.Mask) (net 4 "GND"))
  (pad "2" thru_hole oval locked (at 0 2.54 270) (size 1.7 1.7) (drill 1) (layers *.Cu *.Mask) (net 11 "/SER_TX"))
  (pad "3" thru_hole oval locked (at 0 5.08 270) (size 1.7 1.7) (drill 1) (layers *.Cu *.Mask) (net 12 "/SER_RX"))
  (pad "4" thru_hole oval locked (at 0 7.62 270) (size 1.7 1.7) (drill 1) (layers *.Cu *.Mask) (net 25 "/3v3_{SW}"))
  (pad "5" thru_hole oval locked (at 0 10.16 270) (size 1.7 1.7) (drill 1) (layers *.Cu *.Mask) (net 24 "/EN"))
  (pad "6" thru_hole oval locked (at 0 12.7 270) (size 1.7 1.7) (drill 1) (layers *.Cu *.Mask) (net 23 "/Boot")))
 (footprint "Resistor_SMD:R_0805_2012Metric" (layer "F.Cu") (at 146.685 45.72)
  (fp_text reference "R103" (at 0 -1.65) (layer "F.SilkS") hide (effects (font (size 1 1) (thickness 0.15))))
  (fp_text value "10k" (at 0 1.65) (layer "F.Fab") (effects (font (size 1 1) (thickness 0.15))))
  (fp_line (start -0.227064 -0.735) (end 0.227064 -0.735) (layer "F.SilkS") (width 0.12))
  (fp_line (start -0.227064 0.735) (end 0.227064 0.735) (layer "F.SilkS") (width 0.12))
  (pad "1" smd roundrect locked (at -0.9125 0) (size 1.025 1.4) (layers "F.Cu" "F.Paste" "F.Mask") (roundrect_rratio 0.243902)
   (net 22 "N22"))
  (pad "2" smd roundrect locked (at 0.9125 0) (size 1.025 1.4) (layers "F.Cu" "F.Paste" "F.Mask") (roundrect_rratio 0.243902)
   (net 19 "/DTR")))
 (gr_arc (start 135.255 54.61) (mid 134.356974 54.238026) (end 133.985 53.34) (layer "Edge.Cuts") (width 0.1))
 (gr_line (start 153.162 53.34) (end 153.162 37.465) (layer "Edge.Cuts") (width 0.1))
 (gr_arc (start 153.162 53.34) (mid 152.790026 54.238026) (end 151.892 54.61) (layer "Edge.Cuts") (width 0.1))
 (gr_line (start 124.46 52.07) (end 132.715 52.07) (layer "Edge.Cuts") (width 0.1))
 (gr_line (start 151.892 36.195) (end 124.46 36.195) (layer "Edge.Cuts") (width 0.1))
 (gr_line (start 123.19 37.465) (end 123.19 50.8) (layer "Edge.Cuts") (width 0.1))
 (gr_arc (start 124.46 52.07) (mid 123.561974 51.698026) (end 123.19 50.8) (layer "Edge.Cuts") (width 0.1))
 (gr_arc (start 123.19 37.465) (mid 123.561974 36.566974) (end 124.46 36.195) (layer "Edge.Cuts") (width 0.1))
 (gr_line (start 135.255 54.61) (end 151.892 54.61) (layer "Edge.Cuts") (width 0.1))
 (gr_arc (start 151.892 36.195) (mid 152.790026 36.566974) (end 153.162 37.465) (layer "Edge.Cuts") (width 0.1))
 (gr_arc (start 132.715 52.07) (mid 133.613026 52.441974) (end 133.985 53.34) (layer "Edge.Cuts") (width 0.1))
 (segment (start 131.045 46.105) (end 131.83 46.105) (width 0.2) (layer "F.Cu") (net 9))
 (segment (start 131.045 47.105) (end 131.838 47.105) (width 0.2) (layer "F.Cu") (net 9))
 (segment (start 132.08 46.863) (end 132.08 46.355) (width 0.2) (layer "F.Cu") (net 9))
 (segment (start 131.838 47.105) (end 132.08 46.863) (width 0.2) (layer "F.Cu") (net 9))
 (segment (start 131.83 46.105) (end 132.08 46.355) (width 0.2) (layer "F.Cu") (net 9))
 (segment (start 131.045 45.605) (end 130.163 45.605) (width 0.2) (layer "F.Cu") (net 5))
 (segment (start 129.921 45.847) (end 129.921 46.355) (width 0.2) (layer "F.Cu") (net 5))
 (segment (start 130.163 45.605) (end 129.921 45.847) (width 0.2) (layer "F.Cu") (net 5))
 (segment (start 130.171 46.605) (end 129.921 46.355) (width 0.2) (layer "F.Cu") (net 5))
 (segment (start 131.045 46.605) (end 130.171 46.605) (width 0.2) (layer "F.Cu") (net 5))
 (segment (start 140.716 42.418) (end 139.954 41.656) (width 0.127) (layer "F.Cu") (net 11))
 (segment (start 139.954 40.894) (end 139.7 40.64) (width 0.127) (layer "F.Cu") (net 11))
 (segment (start 140.716 47.879) (end 140.716 42.418) (width 0.127) (layer "F.Cu") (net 11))
 (segment (start 147.32 50.8) (end 146.177 49.657) (width 0.127) (layer "F.Cu") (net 11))
 (segment (start 144.272 49.657) (end 143.891 49.276) (width 0.127) (layer "F.Cu") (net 11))
 (segment (start 139.7 40.64) (end 138.495 40.64) (width 0.127) (layer "F.Cu") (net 11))
 (segment (start 142.113 49.276) (end 140.716 47.879) (width 0.127) (layer "F.Cu") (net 11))
 (segment (start 143.891 49.276) (end 142.113 49.276) (width 0.127) (layer "F.Cu") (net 11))
 (segment (start 146.177 49.657) (end 144.272 49.657) (width 0.127) (layer "F.Cu") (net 11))
 (segment (start 139.954 41.656) (end 139.954 40.894) (width 0.127) (layer "F.Cu") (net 11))
 (segment (start 140.335 42.545) (end 139.7 41.91) (width 0.127) (layer "F.Cu") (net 12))
 (segment (start 141.912201 49.657) (end 140.335 48.079799) (width 0.127) (layer "F.Cu") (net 12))
 (segment (start 140.335 48.079799) (end 140.335 42.545) (width 0.127) (layer "F.Cu") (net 12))
 (segment (start 139.7 41.91) (end 138.495 41.91) (width 0.127) (layer "F.Cu") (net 12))
 (segment (start 144.78 50.8) (end 143.637 49.657) (width 0.127) (layer "F.Cu") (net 12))
 (segment (start 143.637 49.657) (end 141.912201 49.657) (width 0.127) (layer "F.Cu") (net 12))
 (segment (start 145.735 43.195) (end 145.735 43.749) (width 0.127) (layer "F.Cu") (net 24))
 (via (at 145.735 43.749) (size 0.6) (drill 0.3) (layers "F.Cu" "B.Cu") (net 24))
 (segment (start 139.7 48.768) (end 139.7 50.8) (width 0.127) (layer "B.Cu") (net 24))
 (segment (start 145.735 43.749) (end 144.719 43.749) (width 0.127) (layer "B.Cu") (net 24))
 (segment (start 144.719 43.749) (end 139.7 48.768) (width 0.127) (layer "B.Cu") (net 24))
 (segment (start 147.635 41.895) (end 147.635 41.341) (width 0.127) (layer "F.Cu") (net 23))
 (via (at 147.635 41.341) (size 0.6) (drill 0.3) (layers "F.Cu" "B.Cu") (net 23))
 (segment (start 137.16 50.8) (end 146.619 41.341) (width 0.127) (layer "B.Cu") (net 23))
 (segment (start 146.619 41.341) (end 147.635 41.341) (width 0.127) (layer "B.Cu") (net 23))
 (segment (start 144.653 41.91) (end 145.7725 40.7905) (width 0.127) (layer "F.Cu") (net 2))
 (segment (start 148.463 42.926) (end 148.194 43.195) (width 0.127) (layer "F.Cu") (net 2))
 (segment (start 145.7725 39.1395) (end 146.558 38.354) (width 0.127) (layer "F.Cu") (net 2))
 (segment (start 145.7725 40.7905) (end 145.7725 39.37) (width 0.127) (layer "F.Cu") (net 2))
 (segment (start 145.7725 39.37) (end 145.7725 39.1395) (width 0.127) (layer "F.Cu") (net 2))
 (segment (start 148.463 38.735) (end 148.463 42.926) (width 0.127) (layer "F.Cu") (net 2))
 (segment (start 148.194 43.195) (end 147.635 43.195) (width 0.127) (layer "F.Cu") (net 2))
 (segment (start 148.082 38.354) (end 148.463 38.735) (width 0.127) (layer "F.Cu") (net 2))
 (segment (start 146.558 38.354) (end 148.082 38.354) (width 0.127) (layer "F.Cu") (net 2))
 (segment (start 143.445 41.91) (end 143.46 41.895) (width 0.127) (layer "F.Cu") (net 2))
 (segment (start 143.445 41.91) (end 144.653 41.91) (width 0.127) (layer "F.Cu") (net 2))
 (segment (start 147.5975 40.2355) (end 147.5975 39.37) (width 0.127) (layer "F.Cu") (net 1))
 (segment (start 146.304 42.545) (end 146.558 42.291) (width 0.127) (layer "F.Cu") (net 1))
 (segment (start 145.735 42.545) (end 146.304 42.545) (width 0.127) (layer "F.Cu") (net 1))
 (segment (start 146.558 42.291) (end 146.558 41.275) (width 0.127) (layer "F.Cu") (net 1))
 (segment (start 146.558 41.275) (end 147.5975 40.2355) (width 0.127) (layer "F.Cu") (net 1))
 (segment (start 146.939 42.799) (end 147.193 42.545) (width 0.127) (layer "F.Cu") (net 22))
 (segment (start 145.7725 45.4895) (end 146.939 44.323) (width 0.127) (layer "F.Cu") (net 22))
 (segment (start 147.193 42.545) (end 147.635 42.545) (width 0.127) (layer "F.Cu") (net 22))
 (segment (start 145.7725 45.72) (end 145.7725 45.4895) (width 0.127) (layer "F.Cu") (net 22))
 (segment (start 146.939 44.323) (end 146.939 42.799) (width 0.127) (layer "F.Cu") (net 22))
 (segment (start 144.907 43.18) (end 144.907 42.164) (width 0.127) (layer "F.Cu") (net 19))
 (segment (start 147.5975 45.9505) (end 146.812 46.736) (width 0.127) (layer "F.Cu") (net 19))
 (segment (start 145.288 46.736) (end 144.907 46.355) (width 0.127) (layer "F.Cu") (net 19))
 (segment (start 145.176 41.895) (end 144.907 42.164) (width 0.127) (layer "F.Cu") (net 19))
 (segment (start 146.812 46.736) (end 145.288 46.736) (width 0.127) (layer "F.Cu") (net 19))
 (segment (start 145.735 41.895) (end 145.176 41.895) (width 0.127) (layer "F.Cu") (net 19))
 (segment (start 144.907 46.355) (end 144.907 43.18) (width 0.127) (layer "F.Cu") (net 19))
 (segment (start 143.445 43.18) (end 144.907 43.18) (width 0.127) (layer "F.Cu") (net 19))
 (segment (start 147.5975 45.72) (end 147.5975 45.9505) (width 0.127) (layer "F.Cu") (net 19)))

